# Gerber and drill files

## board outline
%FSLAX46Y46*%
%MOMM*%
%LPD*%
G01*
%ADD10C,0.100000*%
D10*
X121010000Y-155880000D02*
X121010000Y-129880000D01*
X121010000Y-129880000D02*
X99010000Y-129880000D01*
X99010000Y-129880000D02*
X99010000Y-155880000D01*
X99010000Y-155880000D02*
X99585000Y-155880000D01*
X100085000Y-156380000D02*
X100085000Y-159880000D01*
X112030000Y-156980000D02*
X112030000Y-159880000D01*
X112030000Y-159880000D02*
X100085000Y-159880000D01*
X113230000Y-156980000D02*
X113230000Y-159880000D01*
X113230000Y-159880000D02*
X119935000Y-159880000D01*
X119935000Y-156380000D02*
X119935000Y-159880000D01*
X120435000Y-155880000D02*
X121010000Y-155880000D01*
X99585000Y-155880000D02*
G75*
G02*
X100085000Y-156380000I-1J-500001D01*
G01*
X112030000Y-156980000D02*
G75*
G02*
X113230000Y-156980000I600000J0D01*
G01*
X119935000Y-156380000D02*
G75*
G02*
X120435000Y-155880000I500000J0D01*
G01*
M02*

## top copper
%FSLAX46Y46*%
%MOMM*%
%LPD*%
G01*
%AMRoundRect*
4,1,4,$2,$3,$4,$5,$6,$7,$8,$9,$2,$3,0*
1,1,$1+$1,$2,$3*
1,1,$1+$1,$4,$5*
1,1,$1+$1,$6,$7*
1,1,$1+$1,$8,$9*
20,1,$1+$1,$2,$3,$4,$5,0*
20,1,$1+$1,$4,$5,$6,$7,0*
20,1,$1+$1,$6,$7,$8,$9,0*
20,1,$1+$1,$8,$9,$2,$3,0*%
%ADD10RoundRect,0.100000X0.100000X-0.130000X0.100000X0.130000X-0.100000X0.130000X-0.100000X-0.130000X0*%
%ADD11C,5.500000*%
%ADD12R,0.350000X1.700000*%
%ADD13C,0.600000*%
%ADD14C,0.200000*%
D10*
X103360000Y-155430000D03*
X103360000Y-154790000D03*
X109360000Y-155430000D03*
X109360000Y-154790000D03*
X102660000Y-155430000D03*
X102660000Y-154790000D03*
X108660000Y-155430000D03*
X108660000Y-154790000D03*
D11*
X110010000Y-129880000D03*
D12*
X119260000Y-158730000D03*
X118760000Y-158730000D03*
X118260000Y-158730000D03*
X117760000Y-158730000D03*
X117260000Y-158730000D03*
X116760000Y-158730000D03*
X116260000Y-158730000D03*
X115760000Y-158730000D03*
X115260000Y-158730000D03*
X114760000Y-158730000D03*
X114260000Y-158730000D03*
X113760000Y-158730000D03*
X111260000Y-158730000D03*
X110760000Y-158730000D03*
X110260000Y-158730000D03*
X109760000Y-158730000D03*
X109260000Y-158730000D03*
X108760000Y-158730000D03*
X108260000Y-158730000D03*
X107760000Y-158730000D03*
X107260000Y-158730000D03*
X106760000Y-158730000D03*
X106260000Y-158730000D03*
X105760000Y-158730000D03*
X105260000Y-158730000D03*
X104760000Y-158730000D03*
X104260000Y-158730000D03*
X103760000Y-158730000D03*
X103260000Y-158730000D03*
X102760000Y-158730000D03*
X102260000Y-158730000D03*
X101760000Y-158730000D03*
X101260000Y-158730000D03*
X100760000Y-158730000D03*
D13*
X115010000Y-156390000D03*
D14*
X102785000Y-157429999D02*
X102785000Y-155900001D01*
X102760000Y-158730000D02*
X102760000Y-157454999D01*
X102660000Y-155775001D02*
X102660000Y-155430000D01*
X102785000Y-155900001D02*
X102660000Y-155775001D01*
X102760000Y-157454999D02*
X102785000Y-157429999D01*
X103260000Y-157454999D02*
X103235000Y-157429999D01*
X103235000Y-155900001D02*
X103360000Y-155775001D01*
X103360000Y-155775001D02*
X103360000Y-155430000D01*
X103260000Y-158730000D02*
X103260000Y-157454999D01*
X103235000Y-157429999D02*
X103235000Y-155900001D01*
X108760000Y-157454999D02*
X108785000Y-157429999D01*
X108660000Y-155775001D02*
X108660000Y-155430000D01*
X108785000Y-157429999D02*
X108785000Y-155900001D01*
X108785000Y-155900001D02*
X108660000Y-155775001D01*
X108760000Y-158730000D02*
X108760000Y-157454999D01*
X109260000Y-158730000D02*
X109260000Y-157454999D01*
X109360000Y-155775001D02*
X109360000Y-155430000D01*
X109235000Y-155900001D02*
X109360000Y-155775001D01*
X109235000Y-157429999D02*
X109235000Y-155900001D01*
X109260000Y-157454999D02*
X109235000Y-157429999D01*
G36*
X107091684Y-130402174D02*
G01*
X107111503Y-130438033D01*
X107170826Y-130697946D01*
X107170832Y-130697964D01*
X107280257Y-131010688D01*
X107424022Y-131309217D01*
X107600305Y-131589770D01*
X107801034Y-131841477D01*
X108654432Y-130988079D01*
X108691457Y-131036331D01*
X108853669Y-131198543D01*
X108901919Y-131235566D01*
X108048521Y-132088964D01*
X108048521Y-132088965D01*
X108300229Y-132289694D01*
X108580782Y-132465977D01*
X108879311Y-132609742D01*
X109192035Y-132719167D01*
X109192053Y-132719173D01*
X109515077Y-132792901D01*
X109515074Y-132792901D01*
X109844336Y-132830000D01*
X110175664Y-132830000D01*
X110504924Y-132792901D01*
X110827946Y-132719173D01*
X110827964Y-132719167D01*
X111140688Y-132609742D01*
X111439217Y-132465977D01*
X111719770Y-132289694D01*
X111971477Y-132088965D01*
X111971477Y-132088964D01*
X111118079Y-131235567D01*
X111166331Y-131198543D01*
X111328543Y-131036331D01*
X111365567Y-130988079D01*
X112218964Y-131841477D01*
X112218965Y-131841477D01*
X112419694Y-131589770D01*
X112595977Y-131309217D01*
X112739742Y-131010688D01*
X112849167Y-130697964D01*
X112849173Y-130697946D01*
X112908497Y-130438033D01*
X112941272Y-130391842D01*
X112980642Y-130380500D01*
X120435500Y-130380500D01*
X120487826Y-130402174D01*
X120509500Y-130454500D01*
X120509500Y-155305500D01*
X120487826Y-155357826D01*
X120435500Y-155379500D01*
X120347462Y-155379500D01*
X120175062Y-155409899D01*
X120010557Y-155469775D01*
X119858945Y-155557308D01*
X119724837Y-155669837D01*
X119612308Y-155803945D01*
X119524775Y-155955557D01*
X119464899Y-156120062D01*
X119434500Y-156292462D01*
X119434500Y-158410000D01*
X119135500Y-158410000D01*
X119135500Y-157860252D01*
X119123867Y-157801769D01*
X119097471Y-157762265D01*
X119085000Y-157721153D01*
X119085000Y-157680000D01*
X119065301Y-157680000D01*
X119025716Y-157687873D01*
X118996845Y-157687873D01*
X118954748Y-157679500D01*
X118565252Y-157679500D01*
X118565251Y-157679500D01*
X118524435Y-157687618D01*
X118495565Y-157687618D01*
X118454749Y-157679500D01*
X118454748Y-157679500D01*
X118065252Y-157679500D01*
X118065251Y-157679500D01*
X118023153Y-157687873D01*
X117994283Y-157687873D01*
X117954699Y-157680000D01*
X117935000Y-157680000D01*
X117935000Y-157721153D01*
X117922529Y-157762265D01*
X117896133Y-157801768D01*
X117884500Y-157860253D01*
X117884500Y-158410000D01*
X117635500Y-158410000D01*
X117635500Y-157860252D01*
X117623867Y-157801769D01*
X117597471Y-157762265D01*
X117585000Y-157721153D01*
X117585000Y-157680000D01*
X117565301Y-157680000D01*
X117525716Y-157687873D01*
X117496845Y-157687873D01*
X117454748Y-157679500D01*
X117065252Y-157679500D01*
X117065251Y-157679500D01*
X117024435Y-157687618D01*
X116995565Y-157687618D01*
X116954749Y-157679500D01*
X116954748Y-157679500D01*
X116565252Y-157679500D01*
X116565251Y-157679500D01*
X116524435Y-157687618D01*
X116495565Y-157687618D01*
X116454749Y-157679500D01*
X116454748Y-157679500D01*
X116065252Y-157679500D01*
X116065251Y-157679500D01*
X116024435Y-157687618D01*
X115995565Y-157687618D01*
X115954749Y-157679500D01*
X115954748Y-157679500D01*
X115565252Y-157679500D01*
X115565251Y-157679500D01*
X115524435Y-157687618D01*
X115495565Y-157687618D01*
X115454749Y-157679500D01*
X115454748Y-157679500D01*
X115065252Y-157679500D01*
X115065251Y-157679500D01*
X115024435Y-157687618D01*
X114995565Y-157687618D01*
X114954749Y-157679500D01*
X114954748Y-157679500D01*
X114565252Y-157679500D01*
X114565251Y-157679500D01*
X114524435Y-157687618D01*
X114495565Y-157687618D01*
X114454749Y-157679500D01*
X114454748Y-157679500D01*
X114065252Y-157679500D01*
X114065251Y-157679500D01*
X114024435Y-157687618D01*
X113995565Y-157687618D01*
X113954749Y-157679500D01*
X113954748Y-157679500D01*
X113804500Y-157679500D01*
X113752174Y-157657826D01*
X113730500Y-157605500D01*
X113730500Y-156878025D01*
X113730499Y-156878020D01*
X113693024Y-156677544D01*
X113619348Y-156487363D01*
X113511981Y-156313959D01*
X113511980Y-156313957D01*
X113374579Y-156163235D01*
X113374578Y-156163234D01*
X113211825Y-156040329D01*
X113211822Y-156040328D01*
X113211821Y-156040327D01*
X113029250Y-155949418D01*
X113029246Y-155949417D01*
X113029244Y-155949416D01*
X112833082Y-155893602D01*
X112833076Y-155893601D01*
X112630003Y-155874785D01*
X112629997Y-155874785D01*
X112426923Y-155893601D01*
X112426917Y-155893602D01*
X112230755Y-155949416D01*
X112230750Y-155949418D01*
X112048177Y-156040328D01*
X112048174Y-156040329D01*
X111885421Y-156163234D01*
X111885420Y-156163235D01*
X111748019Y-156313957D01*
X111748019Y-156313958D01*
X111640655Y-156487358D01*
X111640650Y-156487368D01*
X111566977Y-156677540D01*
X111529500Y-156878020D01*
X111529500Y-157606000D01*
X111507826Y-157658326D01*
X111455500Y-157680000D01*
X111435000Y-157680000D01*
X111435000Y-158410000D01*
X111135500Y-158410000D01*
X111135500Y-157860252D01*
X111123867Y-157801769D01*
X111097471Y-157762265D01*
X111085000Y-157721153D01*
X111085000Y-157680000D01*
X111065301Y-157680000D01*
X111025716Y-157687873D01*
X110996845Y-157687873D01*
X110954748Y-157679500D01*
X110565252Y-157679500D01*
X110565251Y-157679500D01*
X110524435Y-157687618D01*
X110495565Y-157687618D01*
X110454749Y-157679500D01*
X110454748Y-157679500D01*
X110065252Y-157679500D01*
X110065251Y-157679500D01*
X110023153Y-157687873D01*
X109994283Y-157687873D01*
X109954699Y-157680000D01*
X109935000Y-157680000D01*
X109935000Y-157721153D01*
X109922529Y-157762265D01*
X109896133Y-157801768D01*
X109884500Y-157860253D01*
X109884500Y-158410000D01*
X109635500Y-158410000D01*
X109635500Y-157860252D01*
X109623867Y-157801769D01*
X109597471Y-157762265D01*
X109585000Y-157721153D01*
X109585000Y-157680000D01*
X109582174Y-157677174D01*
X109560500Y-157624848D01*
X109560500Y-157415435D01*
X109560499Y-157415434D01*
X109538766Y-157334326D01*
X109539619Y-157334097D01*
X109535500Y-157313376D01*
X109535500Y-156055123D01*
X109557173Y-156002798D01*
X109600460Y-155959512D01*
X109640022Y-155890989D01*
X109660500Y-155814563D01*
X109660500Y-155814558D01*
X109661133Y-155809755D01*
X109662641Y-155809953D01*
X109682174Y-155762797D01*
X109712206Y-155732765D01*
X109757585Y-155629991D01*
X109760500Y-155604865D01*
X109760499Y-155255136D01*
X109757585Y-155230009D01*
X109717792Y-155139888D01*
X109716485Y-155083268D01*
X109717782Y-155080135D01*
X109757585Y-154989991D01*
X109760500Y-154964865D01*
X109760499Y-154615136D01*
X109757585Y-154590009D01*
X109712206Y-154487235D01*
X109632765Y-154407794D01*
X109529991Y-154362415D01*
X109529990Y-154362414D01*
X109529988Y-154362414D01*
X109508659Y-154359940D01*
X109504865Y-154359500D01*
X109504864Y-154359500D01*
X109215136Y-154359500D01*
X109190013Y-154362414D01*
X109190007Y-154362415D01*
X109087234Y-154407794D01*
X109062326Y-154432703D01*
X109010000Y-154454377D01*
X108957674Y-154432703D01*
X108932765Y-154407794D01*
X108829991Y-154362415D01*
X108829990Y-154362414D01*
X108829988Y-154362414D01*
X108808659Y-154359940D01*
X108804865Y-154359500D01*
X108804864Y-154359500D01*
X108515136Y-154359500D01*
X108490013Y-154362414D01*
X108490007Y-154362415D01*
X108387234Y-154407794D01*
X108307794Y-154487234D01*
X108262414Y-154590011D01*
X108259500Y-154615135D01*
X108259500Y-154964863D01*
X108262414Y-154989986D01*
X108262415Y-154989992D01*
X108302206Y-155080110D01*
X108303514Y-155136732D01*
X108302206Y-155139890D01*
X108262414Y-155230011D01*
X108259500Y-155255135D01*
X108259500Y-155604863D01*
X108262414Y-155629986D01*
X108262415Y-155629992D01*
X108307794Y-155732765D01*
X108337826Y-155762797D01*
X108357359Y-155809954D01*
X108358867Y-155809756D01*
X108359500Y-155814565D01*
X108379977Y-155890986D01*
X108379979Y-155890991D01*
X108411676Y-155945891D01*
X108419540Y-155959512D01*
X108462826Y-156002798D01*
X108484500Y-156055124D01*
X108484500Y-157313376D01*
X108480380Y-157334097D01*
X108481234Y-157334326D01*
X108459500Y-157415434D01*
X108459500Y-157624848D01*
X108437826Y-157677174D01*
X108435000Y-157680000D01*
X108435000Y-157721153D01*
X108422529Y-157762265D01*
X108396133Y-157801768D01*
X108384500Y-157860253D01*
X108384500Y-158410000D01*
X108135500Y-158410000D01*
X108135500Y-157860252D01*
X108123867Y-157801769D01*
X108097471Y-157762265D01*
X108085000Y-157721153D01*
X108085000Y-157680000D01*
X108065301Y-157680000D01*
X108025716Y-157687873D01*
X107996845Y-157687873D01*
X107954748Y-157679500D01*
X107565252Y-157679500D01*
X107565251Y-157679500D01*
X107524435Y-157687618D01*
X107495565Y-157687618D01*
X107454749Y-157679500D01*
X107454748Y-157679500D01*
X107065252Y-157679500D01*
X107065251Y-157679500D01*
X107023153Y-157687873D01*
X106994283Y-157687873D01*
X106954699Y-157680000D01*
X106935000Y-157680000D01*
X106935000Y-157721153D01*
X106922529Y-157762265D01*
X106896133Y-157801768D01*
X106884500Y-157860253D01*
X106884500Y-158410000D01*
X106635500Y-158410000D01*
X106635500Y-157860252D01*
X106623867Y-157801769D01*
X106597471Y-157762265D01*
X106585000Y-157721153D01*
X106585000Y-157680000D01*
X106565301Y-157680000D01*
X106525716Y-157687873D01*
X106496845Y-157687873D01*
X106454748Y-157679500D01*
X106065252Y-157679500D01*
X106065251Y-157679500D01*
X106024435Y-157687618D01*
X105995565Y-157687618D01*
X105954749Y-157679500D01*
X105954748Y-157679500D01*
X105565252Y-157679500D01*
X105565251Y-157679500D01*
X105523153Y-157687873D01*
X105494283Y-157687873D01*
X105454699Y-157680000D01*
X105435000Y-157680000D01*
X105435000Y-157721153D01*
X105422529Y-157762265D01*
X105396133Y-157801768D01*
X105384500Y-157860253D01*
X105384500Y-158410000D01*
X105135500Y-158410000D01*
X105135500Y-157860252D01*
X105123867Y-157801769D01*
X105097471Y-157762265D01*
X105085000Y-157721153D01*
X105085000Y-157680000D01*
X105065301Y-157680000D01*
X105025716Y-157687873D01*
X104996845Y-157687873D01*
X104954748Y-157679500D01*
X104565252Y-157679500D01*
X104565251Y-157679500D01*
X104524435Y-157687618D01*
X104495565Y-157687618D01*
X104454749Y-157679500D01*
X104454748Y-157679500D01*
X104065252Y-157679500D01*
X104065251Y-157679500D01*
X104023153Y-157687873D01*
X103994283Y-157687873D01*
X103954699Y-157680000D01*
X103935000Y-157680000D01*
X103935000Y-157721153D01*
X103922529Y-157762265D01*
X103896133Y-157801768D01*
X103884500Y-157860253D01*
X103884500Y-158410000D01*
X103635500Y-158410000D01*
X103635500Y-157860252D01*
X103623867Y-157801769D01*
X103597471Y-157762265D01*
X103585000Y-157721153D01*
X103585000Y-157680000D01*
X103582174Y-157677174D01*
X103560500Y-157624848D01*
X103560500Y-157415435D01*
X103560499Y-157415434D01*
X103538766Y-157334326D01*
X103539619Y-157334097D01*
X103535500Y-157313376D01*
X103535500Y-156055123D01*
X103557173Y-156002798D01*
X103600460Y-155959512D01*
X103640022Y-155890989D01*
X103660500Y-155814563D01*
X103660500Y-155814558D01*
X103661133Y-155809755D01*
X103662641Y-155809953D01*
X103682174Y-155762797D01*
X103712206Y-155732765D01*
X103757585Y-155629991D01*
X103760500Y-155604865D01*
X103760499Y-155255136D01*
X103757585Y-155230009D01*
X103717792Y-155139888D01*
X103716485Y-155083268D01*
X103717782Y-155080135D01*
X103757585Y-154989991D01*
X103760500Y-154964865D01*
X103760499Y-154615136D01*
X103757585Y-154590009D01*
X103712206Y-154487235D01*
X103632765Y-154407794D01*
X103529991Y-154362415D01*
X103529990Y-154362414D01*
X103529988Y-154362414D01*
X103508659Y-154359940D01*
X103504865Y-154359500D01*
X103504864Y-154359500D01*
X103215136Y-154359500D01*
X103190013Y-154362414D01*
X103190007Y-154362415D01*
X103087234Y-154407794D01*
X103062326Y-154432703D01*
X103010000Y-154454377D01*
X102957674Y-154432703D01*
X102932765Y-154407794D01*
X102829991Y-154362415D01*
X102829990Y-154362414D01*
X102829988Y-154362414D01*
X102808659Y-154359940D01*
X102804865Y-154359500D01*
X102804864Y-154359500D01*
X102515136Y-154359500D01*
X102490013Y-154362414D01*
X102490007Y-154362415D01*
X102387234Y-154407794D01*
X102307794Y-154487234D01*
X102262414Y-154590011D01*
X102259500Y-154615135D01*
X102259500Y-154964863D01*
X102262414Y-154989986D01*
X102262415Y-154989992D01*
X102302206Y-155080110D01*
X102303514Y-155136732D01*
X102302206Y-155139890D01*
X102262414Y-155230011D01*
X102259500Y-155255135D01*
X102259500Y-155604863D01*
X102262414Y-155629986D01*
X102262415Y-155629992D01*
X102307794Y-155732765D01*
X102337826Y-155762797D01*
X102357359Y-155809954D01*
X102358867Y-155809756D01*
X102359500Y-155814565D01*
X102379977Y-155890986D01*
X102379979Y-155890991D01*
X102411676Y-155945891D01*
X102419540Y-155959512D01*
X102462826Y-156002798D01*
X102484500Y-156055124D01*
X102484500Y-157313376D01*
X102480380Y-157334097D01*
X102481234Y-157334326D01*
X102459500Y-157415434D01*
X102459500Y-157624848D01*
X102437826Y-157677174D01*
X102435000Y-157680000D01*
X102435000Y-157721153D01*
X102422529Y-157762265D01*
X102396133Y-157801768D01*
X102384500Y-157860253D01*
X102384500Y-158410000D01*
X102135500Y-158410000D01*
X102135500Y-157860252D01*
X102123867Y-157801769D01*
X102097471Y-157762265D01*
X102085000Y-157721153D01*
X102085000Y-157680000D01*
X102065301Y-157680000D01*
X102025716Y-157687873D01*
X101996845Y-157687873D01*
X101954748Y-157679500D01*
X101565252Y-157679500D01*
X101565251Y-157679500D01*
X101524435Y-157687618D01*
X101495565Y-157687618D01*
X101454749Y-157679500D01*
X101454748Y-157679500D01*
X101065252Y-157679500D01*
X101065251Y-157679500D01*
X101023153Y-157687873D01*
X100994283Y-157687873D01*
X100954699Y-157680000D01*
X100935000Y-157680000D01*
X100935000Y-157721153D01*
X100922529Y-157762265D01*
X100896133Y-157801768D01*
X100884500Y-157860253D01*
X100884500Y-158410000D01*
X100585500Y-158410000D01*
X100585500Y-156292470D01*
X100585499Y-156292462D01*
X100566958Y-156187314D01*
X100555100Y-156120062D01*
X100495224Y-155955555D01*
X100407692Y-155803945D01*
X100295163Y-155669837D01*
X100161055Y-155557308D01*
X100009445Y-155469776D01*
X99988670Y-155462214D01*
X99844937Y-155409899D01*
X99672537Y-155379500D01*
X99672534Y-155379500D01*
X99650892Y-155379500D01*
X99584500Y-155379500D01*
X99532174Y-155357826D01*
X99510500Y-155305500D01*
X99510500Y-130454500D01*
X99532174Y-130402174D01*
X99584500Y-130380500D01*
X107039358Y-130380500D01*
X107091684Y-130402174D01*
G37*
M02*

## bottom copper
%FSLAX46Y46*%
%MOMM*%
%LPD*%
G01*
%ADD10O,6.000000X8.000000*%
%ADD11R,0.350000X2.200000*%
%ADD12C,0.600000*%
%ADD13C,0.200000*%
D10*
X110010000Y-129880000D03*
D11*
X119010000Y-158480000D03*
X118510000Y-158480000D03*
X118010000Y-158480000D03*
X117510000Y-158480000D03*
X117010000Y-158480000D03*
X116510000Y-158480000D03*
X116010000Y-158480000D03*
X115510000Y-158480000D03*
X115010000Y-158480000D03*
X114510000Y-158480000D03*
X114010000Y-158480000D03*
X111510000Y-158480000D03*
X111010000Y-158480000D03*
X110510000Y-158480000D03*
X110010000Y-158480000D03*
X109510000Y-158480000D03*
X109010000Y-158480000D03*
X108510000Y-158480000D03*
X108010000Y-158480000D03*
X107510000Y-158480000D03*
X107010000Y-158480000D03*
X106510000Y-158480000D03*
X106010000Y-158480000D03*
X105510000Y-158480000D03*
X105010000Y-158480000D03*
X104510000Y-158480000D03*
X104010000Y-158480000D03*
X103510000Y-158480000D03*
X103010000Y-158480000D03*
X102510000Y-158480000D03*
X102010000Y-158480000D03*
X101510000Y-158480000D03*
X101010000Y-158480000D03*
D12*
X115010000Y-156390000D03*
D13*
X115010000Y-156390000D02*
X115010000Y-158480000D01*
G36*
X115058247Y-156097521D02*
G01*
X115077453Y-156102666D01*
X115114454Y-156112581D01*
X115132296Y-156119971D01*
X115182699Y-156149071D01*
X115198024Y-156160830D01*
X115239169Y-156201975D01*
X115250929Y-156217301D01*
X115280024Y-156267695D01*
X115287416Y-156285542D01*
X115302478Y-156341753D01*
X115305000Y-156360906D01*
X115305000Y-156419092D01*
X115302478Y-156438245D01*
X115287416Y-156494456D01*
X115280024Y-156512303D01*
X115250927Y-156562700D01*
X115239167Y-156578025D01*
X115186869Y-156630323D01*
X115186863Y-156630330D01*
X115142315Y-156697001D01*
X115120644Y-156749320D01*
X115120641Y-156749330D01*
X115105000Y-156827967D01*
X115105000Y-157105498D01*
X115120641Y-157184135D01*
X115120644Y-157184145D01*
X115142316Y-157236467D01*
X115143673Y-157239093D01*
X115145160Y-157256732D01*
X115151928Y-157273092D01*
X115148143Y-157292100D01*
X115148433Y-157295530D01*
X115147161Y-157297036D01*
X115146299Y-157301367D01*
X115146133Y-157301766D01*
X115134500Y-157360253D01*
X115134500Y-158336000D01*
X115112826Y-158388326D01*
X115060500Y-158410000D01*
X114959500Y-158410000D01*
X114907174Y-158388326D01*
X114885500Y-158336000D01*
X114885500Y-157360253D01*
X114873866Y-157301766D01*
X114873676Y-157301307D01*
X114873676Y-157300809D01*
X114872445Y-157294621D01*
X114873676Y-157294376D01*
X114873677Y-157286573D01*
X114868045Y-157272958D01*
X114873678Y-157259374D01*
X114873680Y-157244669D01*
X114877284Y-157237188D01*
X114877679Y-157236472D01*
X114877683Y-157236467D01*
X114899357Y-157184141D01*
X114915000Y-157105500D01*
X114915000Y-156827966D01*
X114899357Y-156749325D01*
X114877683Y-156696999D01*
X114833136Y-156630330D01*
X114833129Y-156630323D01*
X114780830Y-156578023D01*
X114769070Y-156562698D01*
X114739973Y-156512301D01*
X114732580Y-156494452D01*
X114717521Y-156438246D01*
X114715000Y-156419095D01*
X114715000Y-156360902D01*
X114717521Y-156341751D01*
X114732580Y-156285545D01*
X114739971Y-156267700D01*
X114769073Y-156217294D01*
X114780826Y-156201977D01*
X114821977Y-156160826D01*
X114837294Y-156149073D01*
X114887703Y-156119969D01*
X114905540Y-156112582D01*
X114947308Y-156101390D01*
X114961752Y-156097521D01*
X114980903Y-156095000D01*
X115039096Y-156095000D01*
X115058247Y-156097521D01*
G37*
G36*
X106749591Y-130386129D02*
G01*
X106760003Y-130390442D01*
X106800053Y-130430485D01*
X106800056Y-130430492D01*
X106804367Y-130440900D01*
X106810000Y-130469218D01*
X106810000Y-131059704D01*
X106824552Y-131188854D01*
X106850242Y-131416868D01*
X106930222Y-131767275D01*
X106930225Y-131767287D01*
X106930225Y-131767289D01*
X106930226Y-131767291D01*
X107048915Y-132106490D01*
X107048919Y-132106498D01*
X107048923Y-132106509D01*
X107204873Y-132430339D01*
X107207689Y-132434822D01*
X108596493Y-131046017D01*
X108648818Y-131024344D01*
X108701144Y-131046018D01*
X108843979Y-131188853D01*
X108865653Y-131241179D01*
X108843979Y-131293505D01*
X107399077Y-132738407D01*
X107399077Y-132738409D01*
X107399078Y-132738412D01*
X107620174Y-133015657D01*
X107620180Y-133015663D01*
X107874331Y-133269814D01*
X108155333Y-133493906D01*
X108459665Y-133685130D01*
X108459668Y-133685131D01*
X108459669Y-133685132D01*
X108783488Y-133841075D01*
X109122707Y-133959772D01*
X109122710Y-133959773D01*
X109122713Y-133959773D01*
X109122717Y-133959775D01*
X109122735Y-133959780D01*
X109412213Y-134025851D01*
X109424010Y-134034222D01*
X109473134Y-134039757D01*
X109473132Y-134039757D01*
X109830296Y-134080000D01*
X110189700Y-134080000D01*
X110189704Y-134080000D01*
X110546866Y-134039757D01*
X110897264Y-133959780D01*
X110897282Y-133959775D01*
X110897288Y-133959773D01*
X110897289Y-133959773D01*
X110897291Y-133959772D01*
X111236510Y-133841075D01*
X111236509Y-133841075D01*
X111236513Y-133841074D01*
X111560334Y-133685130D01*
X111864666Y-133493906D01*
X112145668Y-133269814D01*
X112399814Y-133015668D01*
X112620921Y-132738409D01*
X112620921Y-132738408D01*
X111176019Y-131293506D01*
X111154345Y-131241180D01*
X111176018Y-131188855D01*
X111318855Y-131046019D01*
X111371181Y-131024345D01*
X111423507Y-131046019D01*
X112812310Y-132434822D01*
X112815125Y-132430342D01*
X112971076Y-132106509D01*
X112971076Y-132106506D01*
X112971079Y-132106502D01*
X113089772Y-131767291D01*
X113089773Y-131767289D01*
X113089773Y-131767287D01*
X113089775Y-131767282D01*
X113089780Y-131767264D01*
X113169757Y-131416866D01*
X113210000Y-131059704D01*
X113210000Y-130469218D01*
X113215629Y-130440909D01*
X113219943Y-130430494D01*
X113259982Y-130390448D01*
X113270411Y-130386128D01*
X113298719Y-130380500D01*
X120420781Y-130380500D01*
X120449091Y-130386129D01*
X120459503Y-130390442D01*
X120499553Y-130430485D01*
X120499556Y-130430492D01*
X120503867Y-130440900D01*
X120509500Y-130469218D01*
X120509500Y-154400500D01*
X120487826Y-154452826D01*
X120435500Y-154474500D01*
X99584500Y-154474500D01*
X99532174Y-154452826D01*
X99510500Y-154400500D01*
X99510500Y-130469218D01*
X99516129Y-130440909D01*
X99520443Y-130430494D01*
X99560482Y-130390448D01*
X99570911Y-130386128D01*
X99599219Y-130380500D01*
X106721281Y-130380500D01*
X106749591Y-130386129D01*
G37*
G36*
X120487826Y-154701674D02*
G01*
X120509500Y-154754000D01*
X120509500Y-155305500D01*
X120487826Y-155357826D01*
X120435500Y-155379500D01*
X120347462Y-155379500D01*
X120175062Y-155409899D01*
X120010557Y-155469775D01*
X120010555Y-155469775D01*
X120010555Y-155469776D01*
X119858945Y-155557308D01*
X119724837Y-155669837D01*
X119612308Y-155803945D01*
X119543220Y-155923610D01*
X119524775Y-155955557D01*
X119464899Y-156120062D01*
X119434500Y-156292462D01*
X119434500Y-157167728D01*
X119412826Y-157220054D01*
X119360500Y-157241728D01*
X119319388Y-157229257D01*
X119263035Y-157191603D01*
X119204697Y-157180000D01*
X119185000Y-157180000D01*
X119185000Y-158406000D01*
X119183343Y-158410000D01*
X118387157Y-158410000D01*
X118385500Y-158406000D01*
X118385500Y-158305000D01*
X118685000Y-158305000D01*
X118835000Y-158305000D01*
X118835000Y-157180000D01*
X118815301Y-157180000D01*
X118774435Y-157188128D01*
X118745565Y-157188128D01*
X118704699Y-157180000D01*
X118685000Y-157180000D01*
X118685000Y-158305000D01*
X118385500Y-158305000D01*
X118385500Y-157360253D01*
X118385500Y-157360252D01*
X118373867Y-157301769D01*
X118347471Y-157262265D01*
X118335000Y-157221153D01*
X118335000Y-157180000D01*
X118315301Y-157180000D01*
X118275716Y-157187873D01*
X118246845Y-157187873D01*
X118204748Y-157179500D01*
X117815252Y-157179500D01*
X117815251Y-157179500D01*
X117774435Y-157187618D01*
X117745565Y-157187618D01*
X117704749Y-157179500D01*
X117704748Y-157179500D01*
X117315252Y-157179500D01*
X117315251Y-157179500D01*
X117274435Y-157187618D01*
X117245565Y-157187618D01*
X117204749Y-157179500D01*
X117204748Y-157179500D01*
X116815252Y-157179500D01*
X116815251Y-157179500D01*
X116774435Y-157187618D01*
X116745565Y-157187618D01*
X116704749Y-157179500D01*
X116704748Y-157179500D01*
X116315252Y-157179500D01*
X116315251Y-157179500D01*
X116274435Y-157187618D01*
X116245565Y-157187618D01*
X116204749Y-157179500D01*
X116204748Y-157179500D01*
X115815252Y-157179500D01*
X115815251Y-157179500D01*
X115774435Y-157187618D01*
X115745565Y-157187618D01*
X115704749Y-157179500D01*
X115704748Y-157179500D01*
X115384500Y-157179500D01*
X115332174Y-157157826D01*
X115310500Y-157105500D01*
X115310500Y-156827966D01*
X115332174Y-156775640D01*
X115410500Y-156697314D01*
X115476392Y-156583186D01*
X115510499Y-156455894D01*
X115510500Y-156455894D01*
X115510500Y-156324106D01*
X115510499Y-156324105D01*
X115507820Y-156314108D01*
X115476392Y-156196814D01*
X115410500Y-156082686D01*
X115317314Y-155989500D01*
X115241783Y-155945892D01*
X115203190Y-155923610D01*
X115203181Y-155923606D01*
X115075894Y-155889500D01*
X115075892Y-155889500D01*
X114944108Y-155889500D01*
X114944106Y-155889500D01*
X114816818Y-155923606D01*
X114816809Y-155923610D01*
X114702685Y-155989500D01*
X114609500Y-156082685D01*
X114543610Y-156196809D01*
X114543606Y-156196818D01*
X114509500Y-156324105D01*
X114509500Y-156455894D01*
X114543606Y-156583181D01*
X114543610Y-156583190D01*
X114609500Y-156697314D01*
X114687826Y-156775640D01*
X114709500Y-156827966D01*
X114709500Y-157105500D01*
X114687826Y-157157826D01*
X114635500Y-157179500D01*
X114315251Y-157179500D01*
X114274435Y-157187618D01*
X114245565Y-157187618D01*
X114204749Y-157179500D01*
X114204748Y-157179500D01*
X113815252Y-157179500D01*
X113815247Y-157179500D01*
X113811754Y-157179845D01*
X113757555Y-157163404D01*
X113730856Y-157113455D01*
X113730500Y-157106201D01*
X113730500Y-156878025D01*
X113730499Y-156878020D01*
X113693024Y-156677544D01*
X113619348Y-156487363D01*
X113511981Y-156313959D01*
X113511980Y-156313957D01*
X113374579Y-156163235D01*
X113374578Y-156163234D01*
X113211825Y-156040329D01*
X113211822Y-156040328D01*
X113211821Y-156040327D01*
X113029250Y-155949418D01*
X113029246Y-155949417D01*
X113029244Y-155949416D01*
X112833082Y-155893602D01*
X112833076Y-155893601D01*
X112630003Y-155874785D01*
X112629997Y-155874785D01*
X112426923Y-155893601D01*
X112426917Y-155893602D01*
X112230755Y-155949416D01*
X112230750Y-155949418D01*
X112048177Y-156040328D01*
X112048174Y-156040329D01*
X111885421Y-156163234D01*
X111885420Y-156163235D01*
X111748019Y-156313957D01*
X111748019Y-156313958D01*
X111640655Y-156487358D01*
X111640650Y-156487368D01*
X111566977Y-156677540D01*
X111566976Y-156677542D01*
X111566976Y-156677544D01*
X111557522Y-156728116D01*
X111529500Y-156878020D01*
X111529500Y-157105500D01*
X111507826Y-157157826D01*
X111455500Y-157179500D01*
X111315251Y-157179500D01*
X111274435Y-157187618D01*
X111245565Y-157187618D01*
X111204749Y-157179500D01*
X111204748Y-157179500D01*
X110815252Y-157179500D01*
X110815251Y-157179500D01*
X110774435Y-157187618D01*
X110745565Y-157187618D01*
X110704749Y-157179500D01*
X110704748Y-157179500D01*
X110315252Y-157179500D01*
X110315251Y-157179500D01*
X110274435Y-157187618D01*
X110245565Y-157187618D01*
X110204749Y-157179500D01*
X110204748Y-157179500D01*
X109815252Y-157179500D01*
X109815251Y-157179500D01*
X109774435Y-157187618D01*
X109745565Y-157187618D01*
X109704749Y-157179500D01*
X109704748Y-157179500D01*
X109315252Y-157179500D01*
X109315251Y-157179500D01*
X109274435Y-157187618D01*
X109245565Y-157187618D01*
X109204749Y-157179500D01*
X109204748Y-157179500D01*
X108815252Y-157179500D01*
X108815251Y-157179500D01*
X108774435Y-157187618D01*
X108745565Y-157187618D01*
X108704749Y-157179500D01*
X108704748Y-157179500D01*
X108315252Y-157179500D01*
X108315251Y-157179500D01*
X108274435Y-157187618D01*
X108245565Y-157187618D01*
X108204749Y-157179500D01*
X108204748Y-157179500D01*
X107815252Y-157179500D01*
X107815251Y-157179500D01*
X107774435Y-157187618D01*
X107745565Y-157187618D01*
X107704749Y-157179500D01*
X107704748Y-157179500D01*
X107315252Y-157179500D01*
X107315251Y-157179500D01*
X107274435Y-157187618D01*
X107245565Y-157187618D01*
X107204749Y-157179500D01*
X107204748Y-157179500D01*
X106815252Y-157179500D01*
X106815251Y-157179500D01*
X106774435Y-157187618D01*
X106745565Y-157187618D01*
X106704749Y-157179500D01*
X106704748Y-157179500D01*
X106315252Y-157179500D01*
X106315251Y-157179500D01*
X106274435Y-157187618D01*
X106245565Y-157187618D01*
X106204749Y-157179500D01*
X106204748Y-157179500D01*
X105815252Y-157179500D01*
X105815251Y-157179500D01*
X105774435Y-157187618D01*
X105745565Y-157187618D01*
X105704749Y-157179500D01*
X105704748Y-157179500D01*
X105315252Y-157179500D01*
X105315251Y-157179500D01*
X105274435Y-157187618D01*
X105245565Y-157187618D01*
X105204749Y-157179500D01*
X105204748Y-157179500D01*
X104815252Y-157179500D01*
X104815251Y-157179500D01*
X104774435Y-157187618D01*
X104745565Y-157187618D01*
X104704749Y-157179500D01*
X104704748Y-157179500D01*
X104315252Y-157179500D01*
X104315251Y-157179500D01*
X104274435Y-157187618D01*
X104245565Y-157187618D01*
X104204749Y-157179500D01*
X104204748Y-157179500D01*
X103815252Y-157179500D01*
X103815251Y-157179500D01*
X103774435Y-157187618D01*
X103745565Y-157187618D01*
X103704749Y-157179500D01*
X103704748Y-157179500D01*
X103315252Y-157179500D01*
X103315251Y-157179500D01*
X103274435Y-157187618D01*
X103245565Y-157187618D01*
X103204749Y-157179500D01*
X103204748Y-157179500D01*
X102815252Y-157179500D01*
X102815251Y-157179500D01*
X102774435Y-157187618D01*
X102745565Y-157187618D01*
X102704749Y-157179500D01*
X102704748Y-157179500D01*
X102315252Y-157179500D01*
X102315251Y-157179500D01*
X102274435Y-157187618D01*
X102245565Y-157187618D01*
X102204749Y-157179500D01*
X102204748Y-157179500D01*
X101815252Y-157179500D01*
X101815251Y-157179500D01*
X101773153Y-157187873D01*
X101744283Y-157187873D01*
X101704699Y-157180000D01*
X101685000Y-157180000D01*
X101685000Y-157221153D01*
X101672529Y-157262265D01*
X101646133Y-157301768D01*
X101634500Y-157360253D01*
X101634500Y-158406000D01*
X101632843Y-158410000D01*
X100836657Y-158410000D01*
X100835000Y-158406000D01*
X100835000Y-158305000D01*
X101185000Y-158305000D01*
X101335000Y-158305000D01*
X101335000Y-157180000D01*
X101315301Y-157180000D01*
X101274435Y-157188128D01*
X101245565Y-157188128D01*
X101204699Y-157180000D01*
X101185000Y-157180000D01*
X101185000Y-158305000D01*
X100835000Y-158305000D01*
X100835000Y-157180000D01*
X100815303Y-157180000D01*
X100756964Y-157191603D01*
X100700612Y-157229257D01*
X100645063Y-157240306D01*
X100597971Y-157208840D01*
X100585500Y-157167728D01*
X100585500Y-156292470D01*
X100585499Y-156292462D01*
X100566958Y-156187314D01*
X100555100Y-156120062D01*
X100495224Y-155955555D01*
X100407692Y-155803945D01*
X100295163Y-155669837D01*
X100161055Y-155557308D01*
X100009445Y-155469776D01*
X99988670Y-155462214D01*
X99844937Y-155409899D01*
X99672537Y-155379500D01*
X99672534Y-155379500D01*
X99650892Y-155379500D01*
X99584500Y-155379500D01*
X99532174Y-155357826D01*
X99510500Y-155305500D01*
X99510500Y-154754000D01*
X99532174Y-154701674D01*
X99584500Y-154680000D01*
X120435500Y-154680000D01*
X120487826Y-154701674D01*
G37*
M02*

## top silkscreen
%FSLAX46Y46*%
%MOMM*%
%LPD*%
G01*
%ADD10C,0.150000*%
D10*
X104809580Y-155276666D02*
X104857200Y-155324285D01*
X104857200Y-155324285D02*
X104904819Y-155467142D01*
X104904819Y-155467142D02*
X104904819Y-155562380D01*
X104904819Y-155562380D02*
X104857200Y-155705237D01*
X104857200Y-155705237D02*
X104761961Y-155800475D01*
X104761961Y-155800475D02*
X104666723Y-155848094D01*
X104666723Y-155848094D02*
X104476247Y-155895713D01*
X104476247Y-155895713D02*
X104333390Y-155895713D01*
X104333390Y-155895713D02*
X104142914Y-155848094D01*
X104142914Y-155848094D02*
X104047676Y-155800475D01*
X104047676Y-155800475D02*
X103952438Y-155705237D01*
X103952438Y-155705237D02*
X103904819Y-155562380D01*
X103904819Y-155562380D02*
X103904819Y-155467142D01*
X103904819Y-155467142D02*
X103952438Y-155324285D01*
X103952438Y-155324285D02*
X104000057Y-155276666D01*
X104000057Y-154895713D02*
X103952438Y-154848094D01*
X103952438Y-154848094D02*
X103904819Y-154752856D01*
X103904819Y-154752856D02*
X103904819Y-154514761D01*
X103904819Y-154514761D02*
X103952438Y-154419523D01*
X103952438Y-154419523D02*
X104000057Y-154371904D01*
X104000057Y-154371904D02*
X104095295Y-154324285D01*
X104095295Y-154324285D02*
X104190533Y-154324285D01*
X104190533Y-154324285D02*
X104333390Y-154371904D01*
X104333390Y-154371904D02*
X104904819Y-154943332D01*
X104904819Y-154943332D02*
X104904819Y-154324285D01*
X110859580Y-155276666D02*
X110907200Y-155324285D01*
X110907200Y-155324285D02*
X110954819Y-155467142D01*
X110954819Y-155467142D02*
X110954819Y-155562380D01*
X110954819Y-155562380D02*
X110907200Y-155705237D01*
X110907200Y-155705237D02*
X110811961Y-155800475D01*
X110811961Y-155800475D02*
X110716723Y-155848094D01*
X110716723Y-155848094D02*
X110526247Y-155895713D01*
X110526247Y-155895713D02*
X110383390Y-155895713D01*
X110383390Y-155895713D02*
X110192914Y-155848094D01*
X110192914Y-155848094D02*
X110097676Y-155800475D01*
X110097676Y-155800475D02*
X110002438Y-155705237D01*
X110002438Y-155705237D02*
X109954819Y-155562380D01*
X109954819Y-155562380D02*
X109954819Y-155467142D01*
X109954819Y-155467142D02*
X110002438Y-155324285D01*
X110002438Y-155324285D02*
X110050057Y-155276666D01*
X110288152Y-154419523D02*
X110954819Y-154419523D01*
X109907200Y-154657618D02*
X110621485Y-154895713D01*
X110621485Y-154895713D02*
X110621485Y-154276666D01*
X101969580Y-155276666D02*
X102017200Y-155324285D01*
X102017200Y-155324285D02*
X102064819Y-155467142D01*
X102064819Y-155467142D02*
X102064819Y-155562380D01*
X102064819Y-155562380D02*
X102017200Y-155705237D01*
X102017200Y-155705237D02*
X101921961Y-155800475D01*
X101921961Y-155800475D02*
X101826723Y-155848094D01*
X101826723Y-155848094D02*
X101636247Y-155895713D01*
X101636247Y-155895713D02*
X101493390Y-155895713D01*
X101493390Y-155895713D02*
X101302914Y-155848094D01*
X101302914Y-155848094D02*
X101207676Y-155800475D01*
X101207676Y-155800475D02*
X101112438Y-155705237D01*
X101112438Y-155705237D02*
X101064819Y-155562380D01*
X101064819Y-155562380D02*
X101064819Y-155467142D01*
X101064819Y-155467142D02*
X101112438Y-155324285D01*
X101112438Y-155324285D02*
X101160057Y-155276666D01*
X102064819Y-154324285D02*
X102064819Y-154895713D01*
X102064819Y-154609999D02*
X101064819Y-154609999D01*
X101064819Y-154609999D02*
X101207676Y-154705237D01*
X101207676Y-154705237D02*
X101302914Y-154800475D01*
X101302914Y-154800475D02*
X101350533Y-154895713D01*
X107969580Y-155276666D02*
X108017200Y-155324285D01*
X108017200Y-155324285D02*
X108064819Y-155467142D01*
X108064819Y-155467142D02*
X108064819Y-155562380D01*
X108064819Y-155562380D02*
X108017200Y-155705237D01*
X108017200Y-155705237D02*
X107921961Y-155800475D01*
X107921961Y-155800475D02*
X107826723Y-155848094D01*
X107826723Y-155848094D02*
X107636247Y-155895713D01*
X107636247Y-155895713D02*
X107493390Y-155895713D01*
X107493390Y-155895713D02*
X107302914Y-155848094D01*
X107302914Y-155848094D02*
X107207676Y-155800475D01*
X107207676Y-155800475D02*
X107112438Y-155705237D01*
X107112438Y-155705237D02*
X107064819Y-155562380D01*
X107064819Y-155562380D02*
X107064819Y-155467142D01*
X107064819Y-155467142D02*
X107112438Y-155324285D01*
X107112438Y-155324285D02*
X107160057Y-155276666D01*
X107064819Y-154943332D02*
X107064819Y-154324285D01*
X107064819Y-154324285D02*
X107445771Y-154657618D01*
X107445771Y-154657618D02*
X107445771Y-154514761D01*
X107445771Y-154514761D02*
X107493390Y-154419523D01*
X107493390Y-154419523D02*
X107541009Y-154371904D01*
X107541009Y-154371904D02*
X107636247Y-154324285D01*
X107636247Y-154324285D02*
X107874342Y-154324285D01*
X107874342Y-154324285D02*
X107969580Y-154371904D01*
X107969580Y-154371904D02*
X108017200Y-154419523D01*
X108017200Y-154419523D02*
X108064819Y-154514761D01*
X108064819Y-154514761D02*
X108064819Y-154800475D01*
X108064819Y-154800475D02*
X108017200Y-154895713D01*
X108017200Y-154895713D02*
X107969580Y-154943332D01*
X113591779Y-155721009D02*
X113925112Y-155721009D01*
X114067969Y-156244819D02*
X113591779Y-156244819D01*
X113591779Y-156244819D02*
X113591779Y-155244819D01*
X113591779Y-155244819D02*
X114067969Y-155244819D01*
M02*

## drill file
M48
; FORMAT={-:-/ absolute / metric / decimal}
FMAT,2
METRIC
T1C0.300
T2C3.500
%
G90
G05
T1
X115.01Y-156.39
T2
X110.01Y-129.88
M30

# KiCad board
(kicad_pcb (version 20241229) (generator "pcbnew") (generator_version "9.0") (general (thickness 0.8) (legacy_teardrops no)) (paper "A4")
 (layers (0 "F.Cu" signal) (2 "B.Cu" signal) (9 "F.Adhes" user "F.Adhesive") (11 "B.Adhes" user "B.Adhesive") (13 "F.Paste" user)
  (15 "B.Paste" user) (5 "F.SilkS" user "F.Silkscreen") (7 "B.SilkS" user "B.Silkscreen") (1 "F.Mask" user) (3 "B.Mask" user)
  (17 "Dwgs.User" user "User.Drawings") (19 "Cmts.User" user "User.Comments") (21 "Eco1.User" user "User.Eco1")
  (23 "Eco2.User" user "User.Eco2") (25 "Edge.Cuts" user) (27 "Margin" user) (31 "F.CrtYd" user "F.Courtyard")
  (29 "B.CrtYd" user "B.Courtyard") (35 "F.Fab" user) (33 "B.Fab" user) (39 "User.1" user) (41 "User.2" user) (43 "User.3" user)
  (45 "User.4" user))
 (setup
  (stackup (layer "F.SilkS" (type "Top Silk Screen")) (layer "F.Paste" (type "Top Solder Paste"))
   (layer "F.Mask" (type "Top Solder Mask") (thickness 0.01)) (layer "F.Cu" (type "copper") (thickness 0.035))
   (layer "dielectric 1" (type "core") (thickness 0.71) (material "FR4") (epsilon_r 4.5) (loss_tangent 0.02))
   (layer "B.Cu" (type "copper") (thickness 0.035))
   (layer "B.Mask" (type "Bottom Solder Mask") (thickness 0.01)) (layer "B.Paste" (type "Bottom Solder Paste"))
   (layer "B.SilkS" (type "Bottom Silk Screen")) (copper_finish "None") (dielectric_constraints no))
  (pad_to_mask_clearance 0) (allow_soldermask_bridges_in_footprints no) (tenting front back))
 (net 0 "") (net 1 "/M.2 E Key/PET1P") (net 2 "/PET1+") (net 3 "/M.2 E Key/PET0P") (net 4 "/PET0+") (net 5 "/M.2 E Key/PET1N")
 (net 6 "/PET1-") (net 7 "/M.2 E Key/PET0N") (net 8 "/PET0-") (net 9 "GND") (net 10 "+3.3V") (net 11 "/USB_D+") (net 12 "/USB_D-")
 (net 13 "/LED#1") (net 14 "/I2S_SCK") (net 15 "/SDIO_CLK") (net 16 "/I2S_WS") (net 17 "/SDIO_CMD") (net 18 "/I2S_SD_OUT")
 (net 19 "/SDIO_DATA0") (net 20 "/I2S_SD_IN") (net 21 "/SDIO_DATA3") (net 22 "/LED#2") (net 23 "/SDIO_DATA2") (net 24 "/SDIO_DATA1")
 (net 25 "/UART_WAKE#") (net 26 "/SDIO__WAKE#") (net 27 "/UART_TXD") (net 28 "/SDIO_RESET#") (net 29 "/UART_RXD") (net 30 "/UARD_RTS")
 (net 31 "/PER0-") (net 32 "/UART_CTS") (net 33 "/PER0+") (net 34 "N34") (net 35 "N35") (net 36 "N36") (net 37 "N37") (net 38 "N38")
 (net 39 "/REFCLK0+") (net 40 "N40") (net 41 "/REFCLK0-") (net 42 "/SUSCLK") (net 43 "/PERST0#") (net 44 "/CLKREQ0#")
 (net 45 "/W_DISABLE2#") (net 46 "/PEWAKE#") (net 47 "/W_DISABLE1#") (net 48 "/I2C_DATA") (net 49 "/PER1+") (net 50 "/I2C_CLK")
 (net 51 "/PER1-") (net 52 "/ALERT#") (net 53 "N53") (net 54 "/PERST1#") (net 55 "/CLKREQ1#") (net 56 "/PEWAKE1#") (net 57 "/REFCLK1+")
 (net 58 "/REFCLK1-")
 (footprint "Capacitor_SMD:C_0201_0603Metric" (layer "F.Cu") (at 103.36 155.11 90)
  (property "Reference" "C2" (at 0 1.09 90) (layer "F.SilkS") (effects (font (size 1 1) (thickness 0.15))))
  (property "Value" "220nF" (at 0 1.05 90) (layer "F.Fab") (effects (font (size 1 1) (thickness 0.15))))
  (pad "" smd roundrect (at -0.345 0 90) (size 0.318 0.36) (layers "F.Paste") (roundrect_rratio 0.25))
  (pad "" smd roundrect (at 0.345 0 90) (size 0.318 0.36) (layers "F.Paste") (roundrect_rratio 0.25))
  (pad "1" smd roundrect (at -0.32 0 90) (size 0.46 0.4) (layers "F.Cu" "F.Mask") (roundrect_rratio 0.25) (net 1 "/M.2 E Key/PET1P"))
  (pad "2" smd roundrect (at 0.32 0 90) (size 0.46 0.4) (layers "F.Cu" "F.Mask") (roundrect_rratio 0.25) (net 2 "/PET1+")))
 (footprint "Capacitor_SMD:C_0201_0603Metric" (layer "F.Cu") (at 109.36 155.11 90)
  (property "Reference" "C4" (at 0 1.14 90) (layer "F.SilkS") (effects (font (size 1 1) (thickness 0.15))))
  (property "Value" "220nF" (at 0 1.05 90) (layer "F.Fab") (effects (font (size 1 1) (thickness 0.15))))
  (pad "" smd roundrect (at -0.345 0 90) (size 0.318 0.36) (layers "F.Paste") (roundrect_rratio 0.25))
  (pad "" smd roundrect (at 0.345 0 90) (size 0.318 0.36) (layers "F.Paste") (roundrect_rratio 0.25))
  (pad "1" smd roundrect (at -0.32 0 90) (size 0.46 0.4) (layers "F.Cu" "F.Mask") (roundrect_rratio 0.25) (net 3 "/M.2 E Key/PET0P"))
  (pad "2" smd roundrect (at 0.32 0 90) (size 0.46 0.4) (layers "F.Cu" "F.Mask") (roundrect_rratio 0.25) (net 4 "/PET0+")))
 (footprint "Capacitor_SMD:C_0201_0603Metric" (layer "F.Cu") (at 102.66 155.11 90)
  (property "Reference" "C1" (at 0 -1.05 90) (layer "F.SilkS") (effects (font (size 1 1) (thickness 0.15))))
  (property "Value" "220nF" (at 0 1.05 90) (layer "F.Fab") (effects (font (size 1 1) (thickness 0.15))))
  (pad "" smd roundrect (at -0.345 0 90) (size 0.318 0.36) (layers "F.Paste") (roundrect_rratio 0.25))
  (pad "" smd roundrect (at 0.345 0 90) (size 0.318 0.36) (layers "F.Paste") (roundrect_rratio 0.25))
  (pad "1" smd roundrect (at -0.32 0 90) (size 0.46 0.4) (layers "F.Cu" "F.Mask") (roundrect_rratio 0.25) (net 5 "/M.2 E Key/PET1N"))
  (pad "2" smd roundrect (at 0.32 0 90) (size 0.46 0.4) (layers "F.Cu" "F.Mask") (roundrect_rratio 0.25) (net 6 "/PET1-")))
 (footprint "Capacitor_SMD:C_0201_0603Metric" (layer "F.Cu") (at 108.66 155.11 90)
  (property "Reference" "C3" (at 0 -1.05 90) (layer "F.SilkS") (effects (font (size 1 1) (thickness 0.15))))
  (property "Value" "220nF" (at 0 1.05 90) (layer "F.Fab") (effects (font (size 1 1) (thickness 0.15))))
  (pad "" smd roundrect (at -0.345 0 90) (size 0.318 0.36) (layers "F.Paste") (roundrect_rratio 0.25))
  (pad "" smd roundrect (at 0.345 0 90) (size 0.318 0.36) (layers "F.Paste") (roundrect_rratio 0.25))
  (pad "1" smd roundrect (at -0.32 0 90) (size 0.46 0.4) (layers "F.Cu" "F.Mask") (roundrect_rratio 0.25) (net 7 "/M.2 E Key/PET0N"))
  (pad "2" smd roundrect (at 0.32 0 90) (size 0.46 0.4) (layers "F.Cu" "F.Mask") (roundrect_rratio 0.25) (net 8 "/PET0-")))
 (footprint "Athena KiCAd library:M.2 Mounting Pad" (layer "F.Cu") (at 110.01 129.88)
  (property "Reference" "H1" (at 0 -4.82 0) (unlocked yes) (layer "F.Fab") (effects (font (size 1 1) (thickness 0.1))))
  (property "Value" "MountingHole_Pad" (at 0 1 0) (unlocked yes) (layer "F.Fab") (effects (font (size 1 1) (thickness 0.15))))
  (pad "1" thru_hole circle (at 0 0) (size 5.5 5.5) (drill 3.5) (layers "*.Cu" "*.Mask") (remove_unused_layers no) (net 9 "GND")
   (padstack (mode front_inner_back)
    (layer "Inner" (shape circle) (size 5.5 5.5) (zone_connect -1))
    (layer "B.Cu" (shape oval) (size 6 8) (thermal_bridge_angle 45) (zone_connect -1)))))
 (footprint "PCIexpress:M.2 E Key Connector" (layer "F.Cu") (at 110.01 158.77)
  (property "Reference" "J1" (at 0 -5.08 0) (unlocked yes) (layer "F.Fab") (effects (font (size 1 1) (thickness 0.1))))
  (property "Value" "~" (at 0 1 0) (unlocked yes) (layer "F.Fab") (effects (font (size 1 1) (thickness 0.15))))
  (fp_line (start -11 -2.89) (end -10.425 -2.89) (stroke (width 0.1) (type default)) (layer "Edge.Cuts"))
  (fp_line (start -9.925 -2.39) (end -9.925 1.11) (stroke (width 0.1) (type default)) (layer "Edge.Cuts"))
  (fp_line (start 2.02 -1.79) (end 2.02 1.11) (stroke (width 0.1) (type default)) (layer "Edge.Cuts"))
  (fp_line (start 2.02 1.11) (end -9.925 1.11) (stroke (width 0.1) (type default)) (layer "Edge.Cuts"))
  (fp_line (start 3.22 -1.79) (end 3.22 1.11) (stroke (width 0.1) (type default)) (layer "Edge.Cuts"))
  (fp_line (start 3.22 1.11) (end 9.925 1.11) (stroke (width 0.1) (type default)) (layer "Edge.Cuts"))
  (fp_line (start 9.925 -2.39) (end 9.925 1.11) (stroke (width 0.1) (type default)) (layer "Edge.Cuts"))
  (fp_line (start 10.425 -2.89) (end 11 -2.89) (stroke (width 0.1) (type default)) (layer "Edge.Cuts"))
  (fp_arc (start -10.425 -2.89) (mid -10.071447 -2.743553) (end -9.925 -2.39) (stroke (width 0.1) (type default)) (layer "Edge.Cuts"))
  (fp_arc (start 2.02 -1.79) (mid 2.62 -2.39) (end 3.22 -1.79) (stroke (width 0.1) (type default)) (layer "Edge.Cuts"))
  (fp_arc (start 9.925 -2.39) (mid 10.071447 -2.743553) (end 10.425 -2.89) (stroke (width 0.1) (type default)) (layer "Edge.Cuts"))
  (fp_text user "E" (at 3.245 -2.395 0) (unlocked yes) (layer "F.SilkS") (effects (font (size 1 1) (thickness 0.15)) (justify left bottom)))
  (pad "1" smd rect (at 9.25 -0.04 180) (size 0.35 1.7) (layers "F.Cu") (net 9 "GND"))
  (pad "2" smd rect (at 9 -0.29 180) (size 0.35 2.2) (layers "B.Cu") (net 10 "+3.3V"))
  (pad "3" smd rect (at 8.75 -0.04 180) (size 0.35 1.7) (layers "F.Cu") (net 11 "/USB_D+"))
  (pad "4" smd rect (at 8.5 -0.29 180) (size 0.35 2.2) (layers "B.Cu") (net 10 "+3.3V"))
  (pad "5" smd rect (at 8.25 -0.04 180) (size 0.35 1.7) (layers "F.Cu") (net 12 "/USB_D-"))
  (pad "6" smd rect (at 8 -0.29 180) (size 0.35 2.2) (layers "B.Cu") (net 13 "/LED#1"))
  (pad "7" smd rect (at 7.75 -0.04 180) (size 0.35 1.7) (layers "F.Cu") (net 9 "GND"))
  (pad "8" smd rect (at 7.5 -0.29 180) (size 0.35 2.2) (layers "B.Cu") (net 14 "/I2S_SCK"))
  (pad "9" smd rect (at 7.25 -0.04 180) (size 0.35 1.7) (layers "F.Cu") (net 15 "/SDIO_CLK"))
  (pad "10" smd rect (at 7 -0.29 180) (size 0.35 2.2) (layers "B.Cu") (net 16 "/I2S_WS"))
  (pad "11" smd rect (at 6.75 -0.04 180) (size 0.35 1.7) (layers "F.Cu") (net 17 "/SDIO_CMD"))
  (pad "12" smd rect (at 6.5 -0.29 180) (size 0.35 2.2) (layers "B.Cu") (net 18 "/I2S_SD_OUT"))
  (pad "13" smd rect (at 6.25 -0.04 180) (size 0.35 1.7) (layers "F.Cu") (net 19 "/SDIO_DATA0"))
  (pad "14" smd rect (at 6 -0.29 180) (size 0.35 2.2) (layers "B.Cu") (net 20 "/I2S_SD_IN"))
  (pad "15" smd rect (at 5.75 -0.04 180) (size 0.35 1.7) (layers "F.Cu") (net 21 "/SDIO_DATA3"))
  (pad "16" smd rect (at 5.5 -0.29 180) (size 0.35 2.2) (layers "B.Cu") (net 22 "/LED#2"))
  (pad "17" smd rect (at 5.25 -0.04 180) (size 0.35 1.7) (layers "F.Cu") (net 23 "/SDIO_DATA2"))
  (pad "18" smd rect (at 5 -0.29 180) (size 0.35 2.2) (layers "B.Cu") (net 9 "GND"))
  (pad "19" smd rect (at 4.75 -0.04 180) (size 0.35 1.7) (layers "F.Cu") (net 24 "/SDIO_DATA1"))
  (pad "20" smd rect (at 4.5 -0.29 180) (size 0.35 2.2) (layers "B.Cu") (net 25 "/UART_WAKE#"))
  (pad "21" smd rect (at 4.25 -0.04 180) (size 0.35 1.7) (layers "F.Cu") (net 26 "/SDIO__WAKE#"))
  (pad "22" smd rect (at 4 -0.29 180) (size 0.35 2.2) (layers "B.Cu") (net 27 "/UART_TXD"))
  (pad "23" smd rect (at 3.75 -0.04 180) (size 0.35 1.7) (layers "F.Cu") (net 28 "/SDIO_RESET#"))
  (pad "32" smd rect (at 1.5 -0.29 180) (size 0.35 2.2) (layers "B.Cu") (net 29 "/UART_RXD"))
  (pad "33" smd rect (at 1.25 -0.04 180) (size 0.35 1.7) (layers "F.Cu") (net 9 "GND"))
  (pad "34" smd rect (at 1 -0.29 180) (size 0.35 2.2) (layers "B.Cu") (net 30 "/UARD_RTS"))
  (pad "35" smd rect (at 0.75 -0.04 180) (size 0.35 1.7) (layers "F.Cu") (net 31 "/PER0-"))
  (pad "36" smd rect (at 0.5 -0.29 180) (size 0.35 2.2) (layers "B.Cu") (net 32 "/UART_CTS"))
  (pad "37" smd rect (at 0.25 -0.04 180) (size 0.35 1.7) (layers "F.Cu") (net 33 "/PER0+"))
  (pad "38" smd rect (at 0 -0.29 180) (size 0.35 2.2) (layers "B.Cu") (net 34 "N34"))
  (pad "39" smd rect (at -0.25 -0.04 180) (size 0.35 1.7) (layers "F.Cu") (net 9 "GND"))
  (pad "40" smd rect (at -0.5 -0.29 180) (size 0.35 2.2) (layers "B.Cu") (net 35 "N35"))
  (pad "41" smd rect (at -0.75 -0.04 180) (size 0.35 1.7) (layers "F.Cu") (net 3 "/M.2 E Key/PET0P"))
  (pad "42" smd rect (at -1 -0.29 180) (size 0.35 2.2) (layers "B.Cu") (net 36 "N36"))
  (pad "43" smd rect (at -1.25 -0.04 180) (size 0.35 1.7) (layers "F.Cu") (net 7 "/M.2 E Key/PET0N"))
  (pad "44" smd rect (at -1.5 -0.29 180) (size 0.35 2.2) (layers "B.Cu") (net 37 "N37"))
  (pad "45" smd rect (at -1.75 -0.04 180) (size 0.35 1.7) (layers "F.Cu") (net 9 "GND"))
  (pad "46" smd rect (at -2 -0.29 180) (size 0.35 2.2) (layers "B.Cu") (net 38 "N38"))
  (pad "47" smd rect (at -2.25 -0.04 180) (size 0.35 1.7) (layers "F.Cu") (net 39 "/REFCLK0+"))
  (pad "48" smd rect (at -2.5 -0.29 180) (size 0.35 2.2) (layers "B.Cu") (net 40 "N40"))
  (pad "49" smd rect (at -2.75 -0.04 180) (size 0.35 1.7) (layers "F.Cu") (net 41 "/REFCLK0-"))
  (pad "50" smd rect (at -3 -0.29 180) (size 0.35 2.2) (layers "B.Cu") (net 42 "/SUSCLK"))
  (pad "51" smd rect (at -3.25 -0.04 180) (size 0.35 1.7) (layers "F.Cu") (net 9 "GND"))
  (pad "52" smd rect (at -3.5 -0.29 180) (size 0.35 2.2) (layers "B.Cu") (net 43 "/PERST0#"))
  (pad "53" smd rect (at -3.75 -0.04 180) (size 0.35 1.7) (layers "F.Cu") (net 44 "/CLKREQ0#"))
  (pad "54" smd rect (at -4 -0.29 180) (size 0.35 2.2) (layers "B.Cu") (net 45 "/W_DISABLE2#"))
  (pad "55" smd rect (at -4.25 -0.04 180) (size 0.35 1.7) (layers "F.Cu") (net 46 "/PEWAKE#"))
  (pad "56" smd rect (at -4.5 -0.29 180) (size 0.35 2.2) (layers "B.Cu") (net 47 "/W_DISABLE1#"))
  (pad "57" smd rect (at -4.75 -0.04 180) (size 0.35 1.7) (layers "F.Cu") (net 9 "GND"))
  (pad "58" smd rect (at -5 -0.29 180) (size 0.35 2.2) (layers "B.Cu") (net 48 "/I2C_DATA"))
  (pad "59" smd rect (at -5.25 -0.04 180) (size 0.35 1.7) (layers "F.Cu") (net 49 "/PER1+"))
  (pad "60" smd rect (at -5.5 -0.29 180) (size 0.35 2.2) (layers "B.Cu") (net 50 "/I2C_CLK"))
  (pad "61" smd rect (at -5.75 -0.04 180) (size 0.35 1.7) (layers "F.Cu") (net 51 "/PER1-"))
  (pad "62" smd rect (at -6 -0.29 180) (size 0.35 2.2) (layers "B.Cu") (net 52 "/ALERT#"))
  (pad "63" smd rect (at -6.25 -0.04 180) (size 0.35 1.7) (layers "F.Cu") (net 9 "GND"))
  (pad "64" smd rect (at -6.5 -0.29 180) (size 0.35 2.2) (layers "B.Cu") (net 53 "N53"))
  (pad "65" smd rect (at -6.75 -0.04 180) (size 0.35 1.7) (layers "F.Cu") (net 1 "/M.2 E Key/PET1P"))
  (pad "66" smd rect (at -7 -0.29 180) (size 0.35 2.2) (layers "B.Cu") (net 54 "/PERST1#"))
  (pad "67" smd rect (at -7.25 -0.04 180) (size 0.35 1.7) (layers "F.Cu") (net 5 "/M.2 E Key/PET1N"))
  (pad "68" smd rect (at -7.5 -0.29 180) (size 0.35 2.2) (layers "B.Cu") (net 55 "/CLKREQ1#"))
  (pad "69" smd rect (at -7.75 -0.04 180) (size 0.35 1.7) (layers "F.Cu") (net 9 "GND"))
  (pad "70" smd rect (at -8 -0.29 180) (size 0.35 2.2) (layers "B.Cu") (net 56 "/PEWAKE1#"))
  (pad "71" smd rect (at -8.25 -0.04 180) (size 0.35 1.7) (layers "F.Cu") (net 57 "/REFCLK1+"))
  (pad "72" smd rect (at -8.5 -0.29 180) (size 0.35 2.2) (layers "B.Cu") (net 10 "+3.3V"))
  (pad "73" smd rect (at -8.75 -0.04 180) (size 0.35 1.7) (layers "F.Cu") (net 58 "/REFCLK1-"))
  (pad "74" smd rect (at -9 -0.29 180) (size 0.35 2.2) (layers "B.Cu") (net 10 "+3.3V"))
  (pad "75" smd rect (at -9.25 -0.04 180) (size 0.35 1.7) (layers "F.Cu") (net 9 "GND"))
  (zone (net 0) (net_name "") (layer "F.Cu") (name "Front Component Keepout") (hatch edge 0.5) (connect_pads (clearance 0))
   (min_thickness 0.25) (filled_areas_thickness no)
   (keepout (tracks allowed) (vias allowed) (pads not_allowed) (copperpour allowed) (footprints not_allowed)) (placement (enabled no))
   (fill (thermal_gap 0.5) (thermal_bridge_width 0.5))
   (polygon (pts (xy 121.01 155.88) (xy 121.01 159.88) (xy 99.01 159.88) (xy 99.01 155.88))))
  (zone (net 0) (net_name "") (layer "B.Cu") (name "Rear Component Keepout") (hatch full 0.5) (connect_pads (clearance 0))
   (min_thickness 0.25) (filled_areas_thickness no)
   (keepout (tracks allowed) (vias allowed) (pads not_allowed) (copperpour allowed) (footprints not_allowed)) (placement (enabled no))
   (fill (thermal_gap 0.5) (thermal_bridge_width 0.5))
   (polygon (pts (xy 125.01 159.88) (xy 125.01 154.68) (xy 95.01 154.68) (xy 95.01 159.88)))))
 (gr_line (start 121.01 155.88) (end 121.01 129.88) (stroke (width 0.1) (type default)) (layer "Edge.Cuts"))
 (gr_line (start 121.01 129.88) (end 99.01 129.88) (stroke (width 0.1) (type default)) (layer "Edge.Cuts"))
 (gr_line (start 99.01 129.88) (end 99.01 155.88) (stroke (width 0.1) (type default)) (layer "Edge.Cuts"))
 (segment (start 102.785 157.429999) (end 102.785 155.900001) (width 0.2) (layer "F.Cu") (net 5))
 (segment (start 102.76 158.73) (end 102.76 157.454999) (width 0.2) (layer "F.Cu") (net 5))
 (segment (start 102.66 155.775001) (end 102.66 155.43) (width 0.2) (layer "F.Cu") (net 5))
 (segment (start 102.785 155.900001) (end 102.66 155.775001) (width 0.2) (layer "F.Cu") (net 5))
 (segment (start 102.76 157.454999) (end 102.785 157.429999) (width 0.2) (layer "F.Cu") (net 5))
 (segment (start 103.26 157.454999) (end 103.235 157.429999) (width 0.2) (layer "F.Cu") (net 1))
 (segment (start 103.235 155.900001) (end 103.36 155.775001) (width 0.2) (layer "F.Cu") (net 1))
 (segment (start 103.36 155.775001) (end 103.36 155.43) (width 0.2) (layer "F.Cu") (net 1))
 (segment (start 103.26 158.73) (end 103.26 157.454999) (width 0.2) (layer "F.Cu") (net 1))
 (segment (start 103.235 157.429999) (end 103.235 155.900001) (width 0.2) (layer "F.Cu") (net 1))
 (segment (start 108.76 157.454999) (end 108.785 157.429999) (width 0.2) (layer "F.Cu") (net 7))
 (segment (start 108.66 155.775001) (end 108.66 155.43) (width 0.2) (layer "F.Cu") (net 7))
 (segment (start 108.785 157.429999) (end 108.785 155.900001) (width 0.2) (layer "F.Cu") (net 7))
 (segment (start 108.785 155.900001) (end 108.66 155.775001) (width 0.2) (layer "F.Cu") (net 7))
 (segment (start 108.76 158.73) (end 108.76 157.454999) (width 0.2) (layer "F.Cu") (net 7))
 (segment (start 109.26 158.73) (end 109.26 157.454999) (width 0.2) (layer "F.Cu") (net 3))
 (segment (start 109.36 155.775001) (end 109.36 155.43) (width 0.2) (layer "F.Cu") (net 3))
 (segment (start 109.235 155.900001) (end 109.36 155.775001) (width 0.2) (layer "F.Cu") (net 3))
 (segment (start 109.235 157.429999) (end 109.235 155.900001) (width 0.2) (layer "F.Cu") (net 3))
 (segment (start 109.26 157.454999) (end 109.235 157.429999) (width 0.2) (layer "F.Cu") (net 3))
 (via (at 115.01 156.39) (size 0.6) (drill 0.3) (layers "F.Cu" "B.Cu") (free yes) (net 9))
 (segment (start 115.01 156.39) (end 115.01 158.48) (width 0.2) (layer "B.Cu") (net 9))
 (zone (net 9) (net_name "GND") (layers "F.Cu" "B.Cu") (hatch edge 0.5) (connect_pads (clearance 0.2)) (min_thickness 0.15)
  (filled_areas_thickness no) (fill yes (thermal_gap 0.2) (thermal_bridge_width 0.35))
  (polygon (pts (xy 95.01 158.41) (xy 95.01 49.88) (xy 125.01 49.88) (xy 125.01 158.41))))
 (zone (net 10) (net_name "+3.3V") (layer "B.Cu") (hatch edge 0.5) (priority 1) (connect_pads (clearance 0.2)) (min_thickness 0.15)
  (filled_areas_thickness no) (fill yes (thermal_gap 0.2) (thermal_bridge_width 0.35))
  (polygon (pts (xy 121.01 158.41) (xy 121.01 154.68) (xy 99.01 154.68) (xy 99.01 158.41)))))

